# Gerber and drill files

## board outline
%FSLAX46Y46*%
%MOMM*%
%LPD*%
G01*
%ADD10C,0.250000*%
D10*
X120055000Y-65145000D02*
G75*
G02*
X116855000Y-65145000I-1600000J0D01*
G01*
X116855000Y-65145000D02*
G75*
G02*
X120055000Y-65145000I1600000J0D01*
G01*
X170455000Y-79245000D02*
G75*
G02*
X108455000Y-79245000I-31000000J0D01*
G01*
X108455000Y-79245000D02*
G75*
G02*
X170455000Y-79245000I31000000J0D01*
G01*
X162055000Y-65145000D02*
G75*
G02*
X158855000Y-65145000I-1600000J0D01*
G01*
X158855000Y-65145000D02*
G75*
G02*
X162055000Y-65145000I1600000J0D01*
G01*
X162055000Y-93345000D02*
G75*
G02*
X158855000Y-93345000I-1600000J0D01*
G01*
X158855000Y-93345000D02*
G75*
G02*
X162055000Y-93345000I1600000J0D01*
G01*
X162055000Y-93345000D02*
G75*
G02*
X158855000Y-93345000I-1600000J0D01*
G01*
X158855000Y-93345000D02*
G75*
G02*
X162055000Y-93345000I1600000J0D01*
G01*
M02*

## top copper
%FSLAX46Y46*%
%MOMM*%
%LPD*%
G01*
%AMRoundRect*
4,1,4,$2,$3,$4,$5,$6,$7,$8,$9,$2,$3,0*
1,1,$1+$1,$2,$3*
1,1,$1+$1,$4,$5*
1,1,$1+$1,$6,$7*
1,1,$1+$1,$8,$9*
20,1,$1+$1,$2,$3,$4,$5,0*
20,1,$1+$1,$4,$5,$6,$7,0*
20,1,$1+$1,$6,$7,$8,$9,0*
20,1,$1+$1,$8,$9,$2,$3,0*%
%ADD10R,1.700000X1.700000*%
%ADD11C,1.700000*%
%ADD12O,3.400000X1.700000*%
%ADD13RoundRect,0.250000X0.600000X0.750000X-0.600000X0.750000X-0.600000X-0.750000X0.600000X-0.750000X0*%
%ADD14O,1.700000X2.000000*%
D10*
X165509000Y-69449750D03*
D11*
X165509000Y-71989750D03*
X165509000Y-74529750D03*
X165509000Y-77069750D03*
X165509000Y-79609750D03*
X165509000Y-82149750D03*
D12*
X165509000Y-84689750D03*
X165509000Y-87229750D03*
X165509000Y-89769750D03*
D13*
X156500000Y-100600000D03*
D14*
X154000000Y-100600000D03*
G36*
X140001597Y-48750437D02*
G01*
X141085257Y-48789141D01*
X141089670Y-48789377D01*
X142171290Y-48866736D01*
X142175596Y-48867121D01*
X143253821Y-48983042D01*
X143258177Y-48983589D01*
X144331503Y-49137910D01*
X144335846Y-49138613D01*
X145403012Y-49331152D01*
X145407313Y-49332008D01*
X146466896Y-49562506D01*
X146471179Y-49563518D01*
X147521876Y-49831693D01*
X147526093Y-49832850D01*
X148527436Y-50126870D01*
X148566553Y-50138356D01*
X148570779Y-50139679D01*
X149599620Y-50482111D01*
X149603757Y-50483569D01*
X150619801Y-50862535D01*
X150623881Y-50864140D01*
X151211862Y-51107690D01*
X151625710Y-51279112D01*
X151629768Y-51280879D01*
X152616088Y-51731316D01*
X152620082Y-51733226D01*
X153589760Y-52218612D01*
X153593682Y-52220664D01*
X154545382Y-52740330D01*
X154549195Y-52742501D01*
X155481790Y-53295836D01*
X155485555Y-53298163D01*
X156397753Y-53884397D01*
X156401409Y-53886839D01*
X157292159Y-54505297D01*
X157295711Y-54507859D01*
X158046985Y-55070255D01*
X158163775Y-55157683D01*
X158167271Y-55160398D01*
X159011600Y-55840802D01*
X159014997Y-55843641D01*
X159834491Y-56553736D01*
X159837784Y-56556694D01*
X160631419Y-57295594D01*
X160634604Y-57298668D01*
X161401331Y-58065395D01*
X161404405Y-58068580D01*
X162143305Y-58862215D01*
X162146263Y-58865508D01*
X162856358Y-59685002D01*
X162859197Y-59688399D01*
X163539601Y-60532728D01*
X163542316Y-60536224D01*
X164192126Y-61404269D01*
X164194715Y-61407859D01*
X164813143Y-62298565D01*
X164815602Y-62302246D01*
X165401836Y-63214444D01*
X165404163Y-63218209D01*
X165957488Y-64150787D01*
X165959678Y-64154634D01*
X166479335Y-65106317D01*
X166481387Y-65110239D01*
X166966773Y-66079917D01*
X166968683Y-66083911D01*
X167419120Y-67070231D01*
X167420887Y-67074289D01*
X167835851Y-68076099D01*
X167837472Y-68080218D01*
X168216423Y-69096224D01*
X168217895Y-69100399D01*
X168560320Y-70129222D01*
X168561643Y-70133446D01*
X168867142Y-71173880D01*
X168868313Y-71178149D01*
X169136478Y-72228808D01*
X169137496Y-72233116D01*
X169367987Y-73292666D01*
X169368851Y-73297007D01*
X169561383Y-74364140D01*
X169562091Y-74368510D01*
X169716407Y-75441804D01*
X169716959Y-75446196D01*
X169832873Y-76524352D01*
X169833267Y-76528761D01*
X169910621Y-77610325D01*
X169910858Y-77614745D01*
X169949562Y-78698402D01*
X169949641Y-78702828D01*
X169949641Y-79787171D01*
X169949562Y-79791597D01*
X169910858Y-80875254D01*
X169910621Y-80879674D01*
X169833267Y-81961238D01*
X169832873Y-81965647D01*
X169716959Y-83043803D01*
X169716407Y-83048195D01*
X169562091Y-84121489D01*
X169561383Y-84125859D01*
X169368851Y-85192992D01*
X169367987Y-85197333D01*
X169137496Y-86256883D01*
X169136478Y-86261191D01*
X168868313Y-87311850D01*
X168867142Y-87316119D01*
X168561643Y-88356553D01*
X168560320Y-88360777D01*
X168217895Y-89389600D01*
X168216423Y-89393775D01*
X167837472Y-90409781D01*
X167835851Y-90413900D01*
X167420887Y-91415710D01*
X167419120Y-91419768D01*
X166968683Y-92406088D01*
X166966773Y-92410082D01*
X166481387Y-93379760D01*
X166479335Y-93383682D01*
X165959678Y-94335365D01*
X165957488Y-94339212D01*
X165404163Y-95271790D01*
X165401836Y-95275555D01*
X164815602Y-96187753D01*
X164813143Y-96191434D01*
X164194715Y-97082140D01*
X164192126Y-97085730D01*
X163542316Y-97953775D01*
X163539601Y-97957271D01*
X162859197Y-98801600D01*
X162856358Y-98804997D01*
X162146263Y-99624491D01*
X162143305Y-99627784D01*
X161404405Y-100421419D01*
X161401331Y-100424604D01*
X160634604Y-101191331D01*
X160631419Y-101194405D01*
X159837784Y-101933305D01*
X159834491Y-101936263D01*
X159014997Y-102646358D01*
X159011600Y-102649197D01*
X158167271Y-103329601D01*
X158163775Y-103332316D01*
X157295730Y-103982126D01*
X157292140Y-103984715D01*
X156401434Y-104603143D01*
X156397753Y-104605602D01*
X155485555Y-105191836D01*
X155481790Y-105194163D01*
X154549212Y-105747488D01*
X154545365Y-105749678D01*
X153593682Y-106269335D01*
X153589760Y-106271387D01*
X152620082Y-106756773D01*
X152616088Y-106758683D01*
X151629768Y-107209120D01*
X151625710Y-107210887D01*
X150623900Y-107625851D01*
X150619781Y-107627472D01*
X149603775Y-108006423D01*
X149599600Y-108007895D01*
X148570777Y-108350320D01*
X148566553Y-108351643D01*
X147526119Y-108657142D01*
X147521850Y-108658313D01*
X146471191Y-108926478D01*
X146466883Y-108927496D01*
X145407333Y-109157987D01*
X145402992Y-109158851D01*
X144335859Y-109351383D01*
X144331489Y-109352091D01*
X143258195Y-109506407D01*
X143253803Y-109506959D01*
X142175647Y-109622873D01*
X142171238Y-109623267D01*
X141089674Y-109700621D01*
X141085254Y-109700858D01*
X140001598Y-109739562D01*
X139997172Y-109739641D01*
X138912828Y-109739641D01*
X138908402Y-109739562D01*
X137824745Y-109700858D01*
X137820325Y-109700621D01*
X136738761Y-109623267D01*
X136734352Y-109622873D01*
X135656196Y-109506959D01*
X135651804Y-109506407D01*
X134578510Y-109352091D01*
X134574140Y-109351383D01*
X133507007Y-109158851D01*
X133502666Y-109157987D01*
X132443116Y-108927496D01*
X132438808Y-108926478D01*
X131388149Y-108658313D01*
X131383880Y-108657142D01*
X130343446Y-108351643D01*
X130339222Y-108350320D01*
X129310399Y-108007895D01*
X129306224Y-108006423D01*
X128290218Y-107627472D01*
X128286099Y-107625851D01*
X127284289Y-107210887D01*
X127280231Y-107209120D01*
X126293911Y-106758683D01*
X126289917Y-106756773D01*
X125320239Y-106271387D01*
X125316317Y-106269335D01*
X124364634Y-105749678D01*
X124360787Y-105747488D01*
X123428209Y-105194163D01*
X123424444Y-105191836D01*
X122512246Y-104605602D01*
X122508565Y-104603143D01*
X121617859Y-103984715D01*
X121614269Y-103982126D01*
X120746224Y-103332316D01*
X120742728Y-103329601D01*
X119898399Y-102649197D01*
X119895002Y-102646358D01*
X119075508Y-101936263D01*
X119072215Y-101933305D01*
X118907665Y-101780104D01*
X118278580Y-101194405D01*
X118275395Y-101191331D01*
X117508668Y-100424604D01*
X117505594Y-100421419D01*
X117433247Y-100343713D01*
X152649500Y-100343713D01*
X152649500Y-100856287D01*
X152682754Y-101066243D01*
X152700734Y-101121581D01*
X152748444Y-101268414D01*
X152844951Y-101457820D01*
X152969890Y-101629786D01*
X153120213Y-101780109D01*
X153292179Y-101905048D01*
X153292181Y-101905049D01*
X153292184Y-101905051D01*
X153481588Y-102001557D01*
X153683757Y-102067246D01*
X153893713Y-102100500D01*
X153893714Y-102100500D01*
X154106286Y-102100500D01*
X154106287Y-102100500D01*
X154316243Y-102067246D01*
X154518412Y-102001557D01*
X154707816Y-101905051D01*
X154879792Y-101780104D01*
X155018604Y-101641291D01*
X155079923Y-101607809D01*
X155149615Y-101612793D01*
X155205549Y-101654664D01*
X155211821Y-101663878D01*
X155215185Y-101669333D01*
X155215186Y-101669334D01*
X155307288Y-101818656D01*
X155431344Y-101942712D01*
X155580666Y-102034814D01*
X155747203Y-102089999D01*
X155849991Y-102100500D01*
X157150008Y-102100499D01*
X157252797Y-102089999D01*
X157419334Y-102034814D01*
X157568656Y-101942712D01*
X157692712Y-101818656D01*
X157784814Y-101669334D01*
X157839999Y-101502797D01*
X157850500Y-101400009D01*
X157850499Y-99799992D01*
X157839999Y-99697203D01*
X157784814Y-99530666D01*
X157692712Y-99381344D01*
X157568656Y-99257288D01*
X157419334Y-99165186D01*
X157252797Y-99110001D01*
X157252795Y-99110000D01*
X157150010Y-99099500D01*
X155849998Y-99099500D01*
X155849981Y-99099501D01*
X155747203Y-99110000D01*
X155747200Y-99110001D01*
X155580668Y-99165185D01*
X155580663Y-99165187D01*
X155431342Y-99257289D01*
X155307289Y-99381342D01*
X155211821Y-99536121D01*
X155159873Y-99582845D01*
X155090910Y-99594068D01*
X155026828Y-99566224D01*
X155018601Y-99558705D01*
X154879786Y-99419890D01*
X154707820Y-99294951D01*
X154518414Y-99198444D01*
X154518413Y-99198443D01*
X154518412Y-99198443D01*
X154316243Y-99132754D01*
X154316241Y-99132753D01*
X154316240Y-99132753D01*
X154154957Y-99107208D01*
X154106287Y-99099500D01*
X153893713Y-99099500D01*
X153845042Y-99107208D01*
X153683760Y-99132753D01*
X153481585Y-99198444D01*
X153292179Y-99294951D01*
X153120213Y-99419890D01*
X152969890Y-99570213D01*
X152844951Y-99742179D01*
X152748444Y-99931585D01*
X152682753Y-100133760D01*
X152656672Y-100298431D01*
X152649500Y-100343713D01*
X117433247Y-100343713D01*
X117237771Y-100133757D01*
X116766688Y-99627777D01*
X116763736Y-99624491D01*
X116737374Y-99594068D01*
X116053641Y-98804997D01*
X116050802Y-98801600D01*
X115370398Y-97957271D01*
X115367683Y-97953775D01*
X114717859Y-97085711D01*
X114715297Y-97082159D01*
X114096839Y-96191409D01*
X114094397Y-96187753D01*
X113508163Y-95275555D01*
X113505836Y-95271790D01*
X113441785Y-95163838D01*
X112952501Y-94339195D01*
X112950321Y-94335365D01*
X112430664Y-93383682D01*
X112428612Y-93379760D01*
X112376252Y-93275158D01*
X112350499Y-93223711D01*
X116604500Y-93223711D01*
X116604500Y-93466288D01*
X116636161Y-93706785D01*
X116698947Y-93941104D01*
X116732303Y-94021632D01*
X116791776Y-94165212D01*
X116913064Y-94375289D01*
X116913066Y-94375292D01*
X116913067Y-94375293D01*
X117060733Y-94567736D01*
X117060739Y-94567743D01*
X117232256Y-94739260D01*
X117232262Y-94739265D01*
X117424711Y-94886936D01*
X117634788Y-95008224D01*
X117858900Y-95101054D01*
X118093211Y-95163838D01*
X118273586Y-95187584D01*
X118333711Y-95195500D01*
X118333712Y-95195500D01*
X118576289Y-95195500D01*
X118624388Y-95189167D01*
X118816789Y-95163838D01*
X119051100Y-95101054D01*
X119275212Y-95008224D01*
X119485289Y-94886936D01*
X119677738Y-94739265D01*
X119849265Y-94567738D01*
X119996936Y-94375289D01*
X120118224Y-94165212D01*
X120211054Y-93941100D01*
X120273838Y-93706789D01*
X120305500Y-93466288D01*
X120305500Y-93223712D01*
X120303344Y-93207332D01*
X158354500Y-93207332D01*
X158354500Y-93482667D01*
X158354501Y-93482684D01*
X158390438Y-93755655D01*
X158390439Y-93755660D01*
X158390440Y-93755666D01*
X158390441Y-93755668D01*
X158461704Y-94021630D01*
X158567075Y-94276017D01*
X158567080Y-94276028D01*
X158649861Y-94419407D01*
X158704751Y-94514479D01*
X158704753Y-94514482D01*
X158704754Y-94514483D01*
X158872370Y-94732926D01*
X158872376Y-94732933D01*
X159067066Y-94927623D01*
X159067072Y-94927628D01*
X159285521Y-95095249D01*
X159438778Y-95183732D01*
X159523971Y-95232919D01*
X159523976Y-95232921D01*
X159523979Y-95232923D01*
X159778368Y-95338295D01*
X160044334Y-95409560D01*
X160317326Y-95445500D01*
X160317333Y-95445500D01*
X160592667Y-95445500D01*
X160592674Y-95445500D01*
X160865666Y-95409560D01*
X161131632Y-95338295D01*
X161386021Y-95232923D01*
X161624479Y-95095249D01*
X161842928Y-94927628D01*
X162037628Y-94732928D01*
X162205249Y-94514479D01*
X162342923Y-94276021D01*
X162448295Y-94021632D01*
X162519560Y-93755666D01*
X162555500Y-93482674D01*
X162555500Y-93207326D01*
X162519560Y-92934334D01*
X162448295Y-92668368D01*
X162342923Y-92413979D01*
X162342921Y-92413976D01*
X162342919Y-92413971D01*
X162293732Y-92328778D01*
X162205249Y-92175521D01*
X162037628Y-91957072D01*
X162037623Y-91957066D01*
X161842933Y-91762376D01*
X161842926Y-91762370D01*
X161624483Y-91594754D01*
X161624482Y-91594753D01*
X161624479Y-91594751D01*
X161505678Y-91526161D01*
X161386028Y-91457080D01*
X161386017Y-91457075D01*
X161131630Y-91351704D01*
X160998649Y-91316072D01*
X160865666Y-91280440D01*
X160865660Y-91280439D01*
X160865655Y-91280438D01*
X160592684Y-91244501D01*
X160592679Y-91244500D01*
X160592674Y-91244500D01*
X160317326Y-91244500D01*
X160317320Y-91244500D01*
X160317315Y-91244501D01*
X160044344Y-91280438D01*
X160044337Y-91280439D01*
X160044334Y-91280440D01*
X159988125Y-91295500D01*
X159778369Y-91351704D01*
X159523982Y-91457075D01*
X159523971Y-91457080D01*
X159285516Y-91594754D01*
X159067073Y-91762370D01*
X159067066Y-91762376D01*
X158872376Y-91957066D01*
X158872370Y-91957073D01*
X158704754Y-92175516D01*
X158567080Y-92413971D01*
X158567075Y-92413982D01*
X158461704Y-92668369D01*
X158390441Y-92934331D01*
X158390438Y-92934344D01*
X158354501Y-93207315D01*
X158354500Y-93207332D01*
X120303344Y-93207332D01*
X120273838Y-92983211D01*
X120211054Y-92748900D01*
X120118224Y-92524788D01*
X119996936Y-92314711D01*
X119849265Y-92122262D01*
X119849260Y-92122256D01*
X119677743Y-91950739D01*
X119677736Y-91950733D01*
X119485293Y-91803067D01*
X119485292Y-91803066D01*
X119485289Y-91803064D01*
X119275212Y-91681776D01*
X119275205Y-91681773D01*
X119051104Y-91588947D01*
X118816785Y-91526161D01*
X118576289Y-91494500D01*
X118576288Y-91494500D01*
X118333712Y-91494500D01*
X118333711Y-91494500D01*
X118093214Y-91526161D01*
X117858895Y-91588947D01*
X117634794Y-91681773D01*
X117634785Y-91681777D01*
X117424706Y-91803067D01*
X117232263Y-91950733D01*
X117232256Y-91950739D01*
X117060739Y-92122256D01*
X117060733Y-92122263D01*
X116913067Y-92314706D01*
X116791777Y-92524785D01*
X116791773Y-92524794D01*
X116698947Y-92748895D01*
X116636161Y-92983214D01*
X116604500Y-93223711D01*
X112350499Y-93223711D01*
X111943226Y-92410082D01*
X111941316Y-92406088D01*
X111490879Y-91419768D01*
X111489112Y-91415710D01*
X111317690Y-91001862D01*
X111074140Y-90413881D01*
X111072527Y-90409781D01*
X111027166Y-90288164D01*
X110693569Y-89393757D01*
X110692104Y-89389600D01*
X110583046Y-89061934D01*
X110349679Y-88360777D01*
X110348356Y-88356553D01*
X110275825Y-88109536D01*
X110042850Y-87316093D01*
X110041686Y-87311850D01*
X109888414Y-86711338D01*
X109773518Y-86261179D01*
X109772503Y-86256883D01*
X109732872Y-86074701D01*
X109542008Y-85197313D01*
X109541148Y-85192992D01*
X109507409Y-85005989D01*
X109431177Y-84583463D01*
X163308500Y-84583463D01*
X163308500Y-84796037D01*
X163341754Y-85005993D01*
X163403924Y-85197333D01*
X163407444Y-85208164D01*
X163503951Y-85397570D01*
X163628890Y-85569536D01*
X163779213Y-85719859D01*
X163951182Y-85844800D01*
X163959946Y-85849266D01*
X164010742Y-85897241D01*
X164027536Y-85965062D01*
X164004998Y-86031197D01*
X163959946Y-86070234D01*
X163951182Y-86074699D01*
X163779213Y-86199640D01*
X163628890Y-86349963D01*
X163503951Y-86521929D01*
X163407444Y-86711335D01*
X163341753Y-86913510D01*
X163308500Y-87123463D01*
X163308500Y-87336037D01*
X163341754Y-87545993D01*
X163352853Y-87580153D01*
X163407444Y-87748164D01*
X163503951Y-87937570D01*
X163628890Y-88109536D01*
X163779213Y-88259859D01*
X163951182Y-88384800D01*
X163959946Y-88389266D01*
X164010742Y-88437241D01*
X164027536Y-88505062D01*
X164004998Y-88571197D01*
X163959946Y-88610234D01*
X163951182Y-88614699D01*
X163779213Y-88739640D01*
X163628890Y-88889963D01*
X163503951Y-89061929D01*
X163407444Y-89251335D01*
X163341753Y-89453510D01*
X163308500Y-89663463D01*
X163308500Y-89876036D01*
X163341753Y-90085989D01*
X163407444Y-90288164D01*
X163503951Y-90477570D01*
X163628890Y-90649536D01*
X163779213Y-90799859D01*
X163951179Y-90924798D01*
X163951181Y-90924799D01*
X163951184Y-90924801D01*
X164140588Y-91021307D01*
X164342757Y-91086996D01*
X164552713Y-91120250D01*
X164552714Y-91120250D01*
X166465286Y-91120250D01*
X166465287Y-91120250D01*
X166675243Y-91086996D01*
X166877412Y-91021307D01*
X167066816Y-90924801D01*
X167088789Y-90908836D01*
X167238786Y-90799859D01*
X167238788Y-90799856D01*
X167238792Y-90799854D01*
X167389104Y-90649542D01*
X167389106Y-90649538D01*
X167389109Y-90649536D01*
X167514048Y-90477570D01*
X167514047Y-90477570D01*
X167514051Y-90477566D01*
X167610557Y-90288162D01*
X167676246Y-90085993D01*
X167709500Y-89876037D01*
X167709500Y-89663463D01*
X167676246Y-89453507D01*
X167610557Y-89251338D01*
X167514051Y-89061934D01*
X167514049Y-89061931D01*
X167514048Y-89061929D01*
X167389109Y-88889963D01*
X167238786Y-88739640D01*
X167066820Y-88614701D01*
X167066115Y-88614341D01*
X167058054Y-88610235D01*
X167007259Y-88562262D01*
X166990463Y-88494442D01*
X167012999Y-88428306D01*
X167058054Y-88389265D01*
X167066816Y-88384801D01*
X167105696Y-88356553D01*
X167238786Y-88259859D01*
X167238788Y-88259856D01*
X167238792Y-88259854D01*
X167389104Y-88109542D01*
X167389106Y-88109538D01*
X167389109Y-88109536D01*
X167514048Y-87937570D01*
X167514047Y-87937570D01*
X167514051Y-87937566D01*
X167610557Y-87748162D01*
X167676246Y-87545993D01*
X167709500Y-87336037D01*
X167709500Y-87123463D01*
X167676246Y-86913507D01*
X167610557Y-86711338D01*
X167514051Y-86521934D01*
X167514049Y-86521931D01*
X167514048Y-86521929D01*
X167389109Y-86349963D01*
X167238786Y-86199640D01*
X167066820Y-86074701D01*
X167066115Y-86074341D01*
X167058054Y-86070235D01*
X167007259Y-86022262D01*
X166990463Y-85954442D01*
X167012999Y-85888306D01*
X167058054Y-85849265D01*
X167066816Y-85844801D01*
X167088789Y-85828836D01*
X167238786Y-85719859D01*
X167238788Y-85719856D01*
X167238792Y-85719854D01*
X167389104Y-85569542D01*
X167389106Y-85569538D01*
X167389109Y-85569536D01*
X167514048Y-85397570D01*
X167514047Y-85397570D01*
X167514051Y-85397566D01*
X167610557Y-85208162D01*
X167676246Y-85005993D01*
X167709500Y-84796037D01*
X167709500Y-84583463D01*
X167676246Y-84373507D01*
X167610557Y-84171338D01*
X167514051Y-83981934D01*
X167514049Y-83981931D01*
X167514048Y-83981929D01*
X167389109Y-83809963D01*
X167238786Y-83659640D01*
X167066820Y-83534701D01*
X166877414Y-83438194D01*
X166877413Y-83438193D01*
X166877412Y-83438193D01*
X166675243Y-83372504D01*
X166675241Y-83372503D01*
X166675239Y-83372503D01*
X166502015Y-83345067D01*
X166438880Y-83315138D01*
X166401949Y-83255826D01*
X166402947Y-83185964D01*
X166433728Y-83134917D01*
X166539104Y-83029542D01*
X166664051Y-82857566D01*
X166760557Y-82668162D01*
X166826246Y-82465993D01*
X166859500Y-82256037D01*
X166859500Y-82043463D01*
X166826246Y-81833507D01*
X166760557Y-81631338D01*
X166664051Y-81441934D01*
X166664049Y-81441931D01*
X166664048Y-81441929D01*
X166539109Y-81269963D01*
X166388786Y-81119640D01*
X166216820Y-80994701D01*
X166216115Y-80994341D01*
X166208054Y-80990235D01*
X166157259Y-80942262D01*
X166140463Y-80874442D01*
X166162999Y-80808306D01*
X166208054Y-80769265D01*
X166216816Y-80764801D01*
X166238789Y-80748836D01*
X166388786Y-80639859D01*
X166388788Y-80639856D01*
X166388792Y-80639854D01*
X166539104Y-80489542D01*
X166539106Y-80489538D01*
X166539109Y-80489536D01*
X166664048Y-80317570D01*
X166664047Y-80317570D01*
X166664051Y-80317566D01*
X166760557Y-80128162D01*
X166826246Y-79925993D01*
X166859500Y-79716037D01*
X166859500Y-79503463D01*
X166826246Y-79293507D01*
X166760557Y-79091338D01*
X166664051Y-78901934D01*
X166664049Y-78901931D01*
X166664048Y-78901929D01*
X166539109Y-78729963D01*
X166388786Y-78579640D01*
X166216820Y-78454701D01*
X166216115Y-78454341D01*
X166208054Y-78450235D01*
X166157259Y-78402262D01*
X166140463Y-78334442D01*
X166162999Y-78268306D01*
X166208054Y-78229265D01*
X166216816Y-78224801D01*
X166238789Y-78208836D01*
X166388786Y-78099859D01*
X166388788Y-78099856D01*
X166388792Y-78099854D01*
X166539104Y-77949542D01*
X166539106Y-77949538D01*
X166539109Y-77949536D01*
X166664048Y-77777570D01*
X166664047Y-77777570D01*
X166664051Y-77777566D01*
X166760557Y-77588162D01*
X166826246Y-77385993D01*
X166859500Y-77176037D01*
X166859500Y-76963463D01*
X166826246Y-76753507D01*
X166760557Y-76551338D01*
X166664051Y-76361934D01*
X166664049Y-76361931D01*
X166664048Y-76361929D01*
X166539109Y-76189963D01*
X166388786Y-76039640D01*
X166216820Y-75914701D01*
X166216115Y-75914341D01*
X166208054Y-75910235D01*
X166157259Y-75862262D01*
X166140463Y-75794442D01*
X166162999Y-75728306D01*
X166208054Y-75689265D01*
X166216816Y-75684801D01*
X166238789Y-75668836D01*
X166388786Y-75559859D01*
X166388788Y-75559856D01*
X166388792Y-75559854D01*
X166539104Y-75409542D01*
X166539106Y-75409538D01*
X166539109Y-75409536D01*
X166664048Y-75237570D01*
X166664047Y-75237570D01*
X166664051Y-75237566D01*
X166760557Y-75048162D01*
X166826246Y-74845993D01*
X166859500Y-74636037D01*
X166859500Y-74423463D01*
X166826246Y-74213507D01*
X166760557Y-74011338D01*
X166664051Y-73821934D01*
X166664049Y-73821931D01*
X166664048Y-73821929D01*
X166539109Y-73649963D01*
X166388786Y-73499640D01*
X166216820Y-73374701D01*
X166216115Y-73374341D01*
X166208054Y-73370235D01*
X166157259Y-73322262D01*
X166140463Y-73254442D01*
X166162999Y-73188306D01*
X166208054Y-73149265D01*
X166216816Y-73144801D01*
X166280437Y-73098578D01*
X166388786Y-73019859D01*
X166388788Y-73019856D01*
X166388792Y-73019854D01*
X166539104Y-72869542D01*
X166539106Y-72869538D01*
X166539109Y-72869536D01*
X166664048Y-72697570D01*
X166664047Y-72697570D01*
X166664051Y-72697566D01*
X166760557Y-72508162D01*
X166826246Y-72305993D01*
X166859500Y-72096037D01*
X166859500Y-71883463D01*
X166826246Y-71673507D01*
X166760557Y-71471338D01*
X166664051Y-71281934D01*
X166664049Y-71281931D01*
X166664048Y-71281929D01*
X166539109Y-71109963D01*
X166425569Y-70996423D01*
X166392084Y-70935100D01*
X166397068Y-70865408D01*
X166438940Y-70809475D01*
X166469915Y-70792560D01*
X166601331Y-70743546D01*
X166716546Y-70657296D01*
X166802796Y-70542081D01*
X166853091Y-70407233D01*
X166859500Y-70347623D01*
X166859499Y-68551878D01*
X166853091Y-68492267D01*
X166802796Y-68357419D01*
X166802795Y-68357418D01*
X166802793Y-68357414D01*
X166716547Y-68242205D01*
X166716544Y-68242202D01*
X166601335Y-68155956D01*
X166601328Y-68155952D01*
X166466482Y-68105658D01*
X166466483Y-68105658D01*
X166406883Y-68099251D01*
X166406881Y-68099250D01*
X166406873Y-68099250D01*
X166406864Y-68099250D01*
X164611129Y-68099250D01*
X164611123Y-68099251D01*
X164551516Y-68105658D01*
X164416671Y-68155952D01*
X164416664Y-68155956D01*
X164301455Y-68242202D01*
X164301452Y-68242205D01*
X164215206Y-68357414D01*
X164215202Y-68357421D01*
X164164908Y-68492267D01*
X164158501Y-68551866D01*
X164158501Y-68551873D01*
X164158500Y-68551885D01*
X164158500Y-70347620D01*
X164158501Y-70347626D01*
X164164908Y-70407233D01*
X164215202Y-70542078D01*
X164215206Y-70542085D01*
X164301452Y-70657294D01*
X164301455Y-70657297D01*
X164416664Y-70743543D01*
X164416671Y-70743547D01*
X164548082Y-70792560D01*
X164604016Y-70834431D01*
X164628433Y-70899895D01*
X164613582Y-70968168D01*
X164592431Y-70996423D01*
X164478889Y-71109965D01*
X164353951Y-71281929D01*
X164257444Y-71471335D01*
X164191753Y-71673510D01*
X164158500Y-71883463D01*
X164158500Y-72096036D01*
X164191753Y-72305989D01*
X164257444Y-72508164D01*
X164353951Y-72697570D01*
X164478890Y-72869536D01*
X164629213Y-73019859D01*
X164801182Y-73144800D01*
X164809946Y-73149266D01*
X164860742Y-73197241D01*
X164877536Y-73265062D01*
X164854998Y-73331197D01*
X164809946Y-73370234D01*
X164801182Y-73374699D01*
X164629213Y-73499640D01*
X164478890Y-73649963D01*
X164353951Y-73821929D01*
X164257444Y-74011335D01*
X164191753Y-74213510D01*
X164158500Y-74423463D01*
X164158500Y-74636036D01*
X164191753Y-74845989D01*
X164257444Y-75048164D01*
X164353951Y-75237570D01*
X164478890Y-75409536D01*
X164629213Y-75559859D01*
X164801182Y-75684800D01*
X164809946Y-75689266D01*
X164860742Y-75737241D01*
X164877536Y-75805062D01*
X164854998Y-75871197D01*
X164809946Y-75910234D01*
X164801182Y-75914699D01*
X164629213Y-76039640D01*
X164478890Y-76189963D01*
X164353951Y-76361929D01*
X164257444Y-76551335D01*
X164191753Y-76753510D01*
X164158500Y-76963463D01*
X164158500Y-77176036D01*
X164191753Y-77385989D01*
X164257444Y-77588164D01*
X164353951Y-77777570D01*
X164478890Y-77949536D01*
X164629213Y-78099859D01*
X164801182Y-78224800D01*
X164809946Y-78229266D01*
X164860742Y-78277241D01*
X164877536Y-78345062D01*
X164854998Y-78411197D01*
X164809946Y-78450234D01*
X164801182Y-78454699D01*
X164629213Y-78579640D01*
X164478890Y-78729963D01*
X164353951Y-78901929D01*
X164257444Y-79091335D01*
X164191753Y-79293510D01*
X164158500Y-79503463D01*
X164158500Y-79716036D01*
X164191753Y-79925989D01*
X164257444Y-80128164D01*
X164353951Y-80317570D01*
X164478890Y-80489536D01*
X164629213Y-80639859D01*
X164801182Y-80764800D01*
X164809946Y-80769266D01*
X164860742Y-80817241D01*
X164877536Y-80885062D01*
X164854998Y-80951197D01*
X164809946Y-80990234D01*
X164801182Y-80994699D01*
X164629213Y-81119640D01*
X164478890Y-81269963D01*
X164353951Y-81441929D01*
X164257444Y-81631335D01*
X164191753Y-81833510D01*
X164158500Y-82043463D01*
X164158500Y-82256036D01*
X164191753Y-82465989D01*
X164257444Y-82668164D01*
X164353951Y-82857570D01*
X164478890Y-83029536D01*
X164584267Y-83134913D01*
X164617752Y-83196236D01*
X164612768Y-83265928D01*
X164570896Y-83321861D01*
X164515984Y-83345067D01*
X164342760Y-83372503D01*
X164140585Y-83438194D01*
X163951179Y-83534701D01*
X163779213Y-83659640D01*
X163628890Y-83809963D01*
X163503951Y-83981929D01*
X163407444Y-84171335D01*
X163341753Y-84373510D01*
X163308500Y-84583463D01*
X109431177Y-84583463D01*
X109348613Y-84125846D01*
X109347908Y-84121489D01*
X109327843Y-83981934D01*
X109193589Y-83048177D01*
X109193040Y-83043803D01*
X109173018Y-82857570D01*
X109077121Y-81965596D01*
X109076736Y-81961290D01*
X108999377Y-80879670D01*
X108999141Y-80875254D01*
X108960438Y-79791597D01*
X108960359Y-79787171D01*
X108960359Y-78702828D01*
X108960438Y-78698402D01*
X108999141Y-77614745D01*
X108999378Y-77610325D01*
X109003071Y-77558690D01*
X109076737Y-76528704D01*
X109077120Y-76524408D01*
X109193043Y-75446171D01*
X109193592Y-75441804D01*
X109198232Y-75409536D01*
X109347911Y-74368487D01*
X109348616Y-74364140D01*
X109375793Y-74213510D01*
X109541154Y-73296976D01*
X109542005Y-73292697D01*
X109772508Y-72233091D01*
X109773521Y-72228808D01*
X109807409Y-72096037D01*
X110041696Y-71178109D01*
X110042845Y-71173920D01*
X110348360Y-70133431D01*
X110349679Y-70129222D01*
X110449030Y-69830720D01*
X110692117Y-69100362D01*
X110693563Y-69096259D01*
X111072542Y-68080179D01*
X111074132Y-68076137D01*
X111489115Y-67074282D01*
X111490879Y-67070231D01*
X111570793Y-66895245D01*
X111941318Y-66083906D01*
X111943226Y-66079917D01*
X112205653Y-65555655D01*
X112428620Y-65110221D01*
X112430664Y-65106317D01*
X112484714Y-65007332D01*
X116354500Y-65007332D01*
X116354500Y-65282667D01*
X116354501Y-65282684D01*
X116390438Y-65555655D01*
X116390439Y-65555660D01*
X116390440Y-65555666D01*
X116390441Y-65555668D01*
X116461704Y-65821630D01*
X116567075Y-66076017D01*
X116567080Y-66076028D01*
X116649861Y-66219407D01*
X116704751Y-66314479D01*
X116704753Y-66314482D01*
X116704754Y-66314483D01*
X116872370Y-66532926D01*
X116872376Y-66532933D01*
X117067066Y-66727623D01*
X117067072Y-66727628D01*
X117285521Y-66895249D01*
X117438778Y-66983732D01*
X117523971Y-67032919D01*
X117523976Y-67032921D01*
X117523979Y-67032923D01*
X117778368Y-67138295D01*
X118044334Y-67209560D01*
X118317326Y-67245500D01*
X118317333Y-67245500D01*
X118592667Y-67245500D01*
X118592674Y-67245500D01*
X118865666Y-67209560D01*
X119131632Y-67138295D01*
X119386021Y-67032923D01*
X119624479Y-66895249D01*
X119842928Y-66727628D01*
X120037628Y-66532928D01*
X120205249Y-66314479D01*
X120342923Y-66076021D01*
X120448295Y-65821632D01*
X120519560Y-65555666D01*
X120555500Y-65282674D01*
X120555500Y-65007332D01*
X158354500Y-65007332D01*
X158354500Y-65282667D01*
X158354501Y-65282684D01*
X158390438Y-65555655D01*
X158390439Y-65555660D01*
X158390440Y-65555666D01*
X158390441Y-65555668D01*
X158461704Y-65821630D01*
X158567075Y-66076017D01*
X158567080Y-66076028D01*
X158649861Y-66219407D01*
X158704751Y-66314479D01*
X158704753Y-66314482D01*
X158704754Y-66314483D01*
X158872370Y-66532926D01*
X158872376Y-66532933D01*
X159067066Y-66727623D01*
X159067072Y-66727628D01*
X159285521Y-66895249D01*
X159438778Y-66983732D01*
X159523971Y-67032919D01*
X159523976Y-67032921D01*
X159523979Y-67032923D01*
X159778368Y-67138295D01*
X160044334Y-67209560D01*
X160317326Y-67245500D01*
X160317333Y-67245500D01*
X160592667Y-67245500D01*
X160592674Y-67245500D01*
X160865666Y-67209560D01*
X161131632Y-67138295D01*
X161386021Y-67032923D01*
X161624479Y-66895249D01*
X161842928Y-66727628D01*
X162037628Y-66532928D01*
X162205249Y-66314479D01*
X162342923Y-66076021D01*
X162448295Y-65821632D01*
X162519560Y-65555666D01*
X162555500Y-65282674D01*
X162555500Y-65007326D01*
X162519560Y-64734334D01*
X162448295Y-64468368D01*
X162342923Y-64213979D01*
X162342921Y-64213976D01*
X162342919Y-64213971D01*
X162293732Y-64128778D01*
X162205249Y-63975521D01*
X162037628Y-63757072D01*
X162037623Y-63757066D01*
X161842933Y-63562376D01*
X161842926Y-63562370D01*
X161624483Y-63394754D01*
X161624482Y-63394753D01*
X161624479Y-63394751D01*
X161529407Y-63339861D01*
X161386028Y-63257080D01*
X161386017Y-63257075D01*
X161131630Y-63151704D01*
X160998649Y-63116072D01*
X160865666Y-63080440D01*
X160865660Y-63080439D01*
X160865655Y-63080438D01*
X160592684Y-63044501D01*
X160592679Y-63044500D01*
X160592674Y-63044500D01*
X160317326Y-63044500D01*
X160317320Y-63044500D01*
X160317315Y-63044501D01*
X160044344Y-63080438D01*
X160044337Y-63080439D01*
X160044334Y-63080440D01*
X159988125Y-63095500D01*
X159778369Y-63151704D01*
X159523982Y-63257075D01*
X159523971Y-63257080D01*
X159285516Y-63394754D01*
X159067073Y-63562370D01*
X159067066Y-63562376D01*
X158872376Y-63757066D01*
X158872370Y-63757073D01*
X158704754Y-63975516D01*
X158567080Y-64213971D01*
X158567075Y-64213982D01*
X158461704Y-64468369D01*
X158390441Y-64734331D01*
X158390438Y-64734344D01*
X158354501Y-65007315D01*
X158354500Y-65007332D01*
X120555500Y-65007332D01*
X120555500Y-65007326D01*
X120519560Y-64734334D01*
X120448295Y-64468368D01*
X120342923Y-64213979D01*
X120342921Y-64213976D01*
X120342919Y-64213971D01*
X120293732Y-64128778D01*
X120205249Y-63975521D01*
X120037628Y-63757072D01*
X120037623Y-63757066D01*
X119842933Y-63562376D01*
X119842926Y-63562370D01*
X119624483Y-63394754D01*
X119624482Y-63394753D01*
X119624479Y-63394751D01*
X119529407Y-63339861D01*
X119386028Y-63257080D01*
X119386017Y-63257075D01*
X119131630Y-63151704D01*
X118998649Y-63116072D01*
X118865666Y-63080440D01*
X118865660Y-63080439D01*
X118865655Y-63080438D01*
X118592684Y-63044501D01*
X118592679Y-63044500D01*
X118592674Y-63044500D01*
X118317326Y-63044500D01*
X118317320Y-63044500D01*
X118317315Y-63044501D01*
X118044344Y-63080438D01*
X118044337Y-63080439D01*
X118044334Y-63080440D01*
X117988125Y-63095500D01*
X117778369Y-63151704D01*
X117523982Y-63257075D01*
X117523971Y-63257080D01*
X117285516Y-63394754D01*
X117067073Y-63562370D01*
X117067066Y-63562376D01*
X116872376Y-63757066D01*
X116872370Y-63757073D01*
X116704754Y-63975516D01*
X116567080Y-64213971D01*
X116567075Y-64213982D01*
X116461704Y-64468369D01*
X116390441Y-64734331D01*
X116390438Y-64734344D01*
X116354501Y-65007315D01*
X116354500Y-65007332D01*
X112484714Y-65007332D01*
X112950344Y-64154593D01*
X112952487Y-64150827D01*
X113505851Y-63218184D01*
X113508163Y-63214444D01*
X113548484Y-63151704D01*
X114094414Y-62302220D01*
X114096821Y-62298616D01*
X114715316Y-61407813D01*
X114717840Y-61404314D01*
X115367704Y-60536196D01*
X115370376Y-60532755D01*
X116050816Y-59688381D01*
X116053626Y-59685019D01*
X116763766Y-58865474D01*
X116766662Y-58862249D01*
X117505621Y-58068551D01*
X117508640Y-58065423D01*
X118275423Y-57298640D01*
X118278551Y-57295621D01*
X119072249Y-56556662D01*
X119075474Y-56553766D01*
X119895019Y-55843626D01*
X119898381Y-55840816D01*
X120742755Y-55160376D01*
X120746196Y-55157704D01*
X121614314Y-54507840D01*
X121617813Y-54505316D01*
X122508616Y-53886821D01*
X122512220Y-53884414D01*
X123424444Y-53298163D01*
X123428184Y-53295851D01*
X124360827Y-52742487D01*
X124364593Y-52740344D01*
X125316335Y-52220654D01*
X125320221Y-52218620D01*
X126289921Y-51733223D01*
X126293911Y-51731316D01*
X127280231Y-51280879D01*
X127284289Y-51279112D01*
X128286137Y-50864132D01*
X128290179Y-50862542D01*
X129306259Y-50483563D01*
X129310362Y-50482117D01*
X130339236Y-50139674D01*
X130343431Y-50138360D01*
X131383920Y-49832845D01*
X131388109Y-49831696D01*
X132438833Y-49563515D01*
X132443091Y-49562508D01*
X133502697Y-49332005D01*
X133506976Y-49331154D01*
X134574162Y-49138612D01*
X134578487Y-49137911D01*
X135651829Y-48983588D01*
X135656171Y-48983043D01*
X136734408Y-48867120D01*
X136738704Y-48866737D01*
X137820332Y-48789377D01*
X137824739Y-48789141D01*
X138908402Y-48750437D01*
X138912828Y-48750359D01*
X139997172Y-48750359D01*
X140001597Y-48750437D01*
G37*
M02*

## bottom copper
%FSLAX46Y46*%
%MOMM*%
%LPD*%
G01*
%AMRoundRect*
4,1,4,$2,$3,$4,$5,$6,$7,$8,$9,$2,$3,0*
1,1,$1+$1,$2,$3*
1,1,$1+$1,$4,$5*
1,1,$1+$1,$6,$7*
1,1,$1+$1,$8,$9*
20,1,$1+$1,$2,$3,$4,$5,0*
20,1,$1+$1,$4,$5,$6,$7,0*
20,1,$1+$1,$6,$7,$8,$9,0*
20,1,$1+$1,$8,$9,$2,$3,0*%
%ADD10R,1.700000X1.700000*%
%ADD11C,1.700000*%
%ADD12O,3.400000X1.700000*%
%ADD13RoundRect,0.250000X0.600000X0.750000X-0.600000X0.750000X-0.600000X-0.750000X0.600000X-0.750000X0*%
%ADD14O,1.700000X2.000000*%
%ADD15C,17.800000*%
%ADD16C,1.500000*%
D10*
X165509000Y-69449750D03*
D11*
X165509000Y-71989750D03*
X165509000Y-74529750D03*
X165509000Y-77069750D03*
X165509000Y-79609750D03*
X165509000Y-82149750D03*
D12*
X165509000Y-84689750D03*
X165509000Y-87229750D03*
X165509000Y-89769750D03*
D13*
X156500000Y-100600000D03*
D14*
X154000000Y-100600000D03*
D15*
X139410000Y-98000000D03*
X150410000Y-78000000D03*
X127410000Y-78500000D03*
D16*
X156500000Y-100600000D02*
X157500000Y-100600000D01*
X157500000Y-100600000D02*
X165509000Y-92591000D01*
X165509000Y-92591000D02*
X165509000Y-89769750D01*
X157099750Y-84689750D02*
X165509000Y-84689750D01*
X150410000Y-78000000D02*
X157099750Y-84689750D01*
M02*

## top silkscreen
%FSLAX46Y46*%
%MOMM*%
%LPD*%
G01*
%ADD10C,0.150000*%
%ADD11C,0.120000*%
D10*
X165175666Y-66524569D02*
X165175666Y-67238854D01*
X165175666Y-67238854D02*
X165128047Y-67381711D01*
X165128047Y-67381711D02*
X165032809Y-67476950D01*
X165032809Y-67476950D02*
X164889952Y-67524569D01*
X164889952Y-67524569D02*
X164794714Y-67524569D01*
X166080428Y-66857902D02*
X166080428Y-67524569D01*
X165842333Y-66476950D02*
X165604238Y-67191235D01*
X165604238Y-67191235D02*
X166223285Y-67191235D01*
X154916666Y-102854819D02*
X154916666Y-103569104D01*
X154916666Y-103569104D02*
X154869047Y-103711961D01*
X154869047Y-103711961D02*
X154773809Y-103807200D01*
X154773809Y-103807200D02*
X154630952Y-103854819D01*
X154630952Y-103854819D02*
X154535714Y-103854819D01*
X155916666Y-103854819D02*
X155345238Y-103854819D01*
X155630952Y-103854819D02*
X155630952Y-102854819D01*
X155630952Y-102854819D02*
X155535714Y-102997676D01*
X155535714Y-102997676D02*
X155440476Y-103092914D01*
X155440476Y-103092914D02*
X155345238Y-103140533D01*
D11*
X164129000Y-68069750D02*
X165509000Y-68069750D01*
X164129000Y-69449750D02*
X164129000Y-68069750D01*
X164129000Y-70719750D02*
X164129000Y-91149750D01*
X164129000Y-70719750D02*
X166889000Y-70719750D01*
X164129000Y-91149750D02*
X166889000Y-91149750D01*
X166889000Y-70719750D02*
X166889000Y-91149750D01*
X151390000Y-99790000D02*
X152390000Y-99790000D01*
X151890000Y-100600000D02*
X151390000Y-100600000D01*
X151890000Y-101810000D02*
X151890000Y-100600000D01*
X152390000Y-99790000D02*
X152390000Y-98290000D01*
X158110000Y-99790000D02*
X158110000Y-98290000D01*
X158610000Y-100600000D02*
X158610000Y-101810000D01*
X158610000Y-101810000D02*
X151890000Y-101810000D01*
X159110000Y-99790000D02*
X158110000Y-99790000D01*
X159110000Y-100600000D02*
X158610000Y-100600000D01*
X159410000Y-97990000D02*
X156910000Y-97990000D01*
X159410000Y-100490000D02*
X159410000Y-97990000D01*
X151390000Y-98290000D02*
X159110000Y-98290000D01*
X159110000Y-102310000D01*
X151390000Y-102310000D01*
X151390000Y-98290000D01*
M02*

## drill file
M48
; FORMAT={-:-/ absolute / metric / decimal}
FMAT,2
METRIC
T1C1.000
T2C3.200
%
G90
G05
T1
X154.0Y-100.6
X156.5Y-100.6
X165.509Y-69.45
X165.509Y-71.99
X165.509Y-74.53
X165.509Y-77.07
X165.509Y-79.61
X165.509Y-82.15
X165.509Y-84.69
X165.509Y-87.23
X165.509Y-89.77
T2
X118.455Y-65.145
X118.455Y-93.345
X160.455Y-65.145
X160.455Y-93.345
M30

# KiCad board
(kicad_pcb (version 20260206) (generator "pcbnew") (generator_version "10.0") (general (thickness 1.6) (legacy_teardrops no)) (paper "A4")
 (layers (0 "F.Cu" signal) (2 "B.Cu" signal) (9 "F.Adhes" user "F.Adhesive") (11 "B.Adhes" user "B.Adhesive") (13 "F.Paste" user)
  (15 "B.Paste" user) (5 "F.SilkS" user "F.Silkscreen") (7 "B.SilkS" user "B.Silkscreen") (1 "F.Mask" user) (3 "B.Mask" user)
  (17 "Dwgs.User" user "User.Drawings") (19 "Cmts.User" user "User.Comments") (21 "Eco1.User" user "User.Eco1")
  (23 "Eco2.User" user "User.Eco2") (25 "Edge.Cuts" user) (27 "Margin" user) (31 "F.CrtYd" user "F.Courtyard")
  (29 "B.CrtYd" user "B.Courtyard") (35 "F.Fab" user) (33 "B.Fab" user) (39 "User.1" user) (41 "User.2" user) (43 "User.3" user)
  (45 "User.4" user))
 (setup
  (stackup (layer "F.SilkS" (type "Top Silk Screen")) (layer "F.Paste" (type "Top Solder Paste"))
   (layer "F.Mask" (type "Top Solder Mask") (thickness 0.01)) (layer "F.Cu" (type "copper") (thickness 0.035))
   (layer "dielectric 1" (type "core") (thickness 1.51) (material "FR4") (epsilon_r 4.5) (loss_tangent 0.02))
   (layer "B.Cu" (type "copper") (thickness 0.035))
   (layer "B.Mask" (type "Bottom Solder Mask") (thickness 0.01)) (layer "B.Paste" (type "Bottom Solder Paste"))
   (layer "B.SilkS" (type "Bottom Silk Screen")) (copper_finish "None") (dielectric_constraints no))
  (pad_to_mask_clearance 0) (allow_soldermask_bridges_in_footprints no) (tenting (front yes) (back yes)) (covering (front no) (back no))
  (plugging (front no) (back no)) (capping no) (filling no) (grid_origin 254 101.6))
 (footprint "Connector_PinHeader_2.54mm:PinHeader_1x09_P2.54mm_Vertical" (layer "F.Cu") (at 165.509 69.44975)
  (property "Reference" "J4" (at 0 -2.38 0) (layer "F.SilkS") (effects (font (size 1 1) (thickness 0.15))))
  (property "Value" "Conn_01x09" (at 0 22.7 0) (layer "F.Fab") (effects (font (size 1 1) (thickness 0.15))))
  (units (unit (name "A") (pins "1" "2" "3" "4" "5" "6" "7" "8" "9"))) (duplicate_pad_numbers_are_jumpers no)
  (fp_line (start -1.38 -1.38) (end 0 -1.38) (stroke (width 0.12) (type solid)) (layer "F.SilkS"))
  (fp_line (start -1.38 0) (end -1.38 -1.38) (stroke (width 0.12) (type solid)) (layer "F.SilkS"))
  (fp_line (start -1.38 1.27) (end -1.38 21.7) (stroke (width 0.12) (type solid)) (layer "F.SilkS"))
  (fp_line (start -1.38 1.27) (end 1.38 1.27) (stroke (width 0.12) (type solid)) (layer "F.SilkS"))
  (fp_line (start -1.38 21.7) (end 1.38 21.7) (stroke (width 0.12) (type solid)) (layer "F.SilkS"))
  (fp_line (start 1.38 1.27) (end 1.38 21.7) (stroke (width 0.12) (type solid)) (layer "F.SilkS"))
  (pad "1" thru_hole rect (at 0 0) (size 1.7 1.7) (drill 1) (layers "*.Cu" "*.Mask") (remove_unused_layers no)
   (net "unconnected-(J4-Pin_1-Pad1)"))
  (pad "2" thru_hole circle (at 0 2.54) (size 1.7 1.7) (drill 1) (layers "*.Cu" "*.Mask") (remove_unused_layers no)
   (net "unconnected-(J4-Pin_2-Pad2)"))
  (pad "3" thru_hole circle (at 0 5.08) (size 1.7 1.7) (drill 1) (layers "*.Cu" "*.Mask") (remove_unused_layers no)
   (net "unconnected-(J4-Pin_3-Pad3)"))
  (pad "4" thru_hole circle (at 0 7.62) (size 1.7 1.7) (drill 1) (layers "*.Cu" "*.Mask") (remove_unused_layers no)
   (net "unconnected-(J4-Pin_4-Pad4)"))
  (pad "5" thru_hole circle (at 0 10.16) (size 1.7 1.7) (drill 1) (layers "*.Cu" "*.Mask") (remove_unused_layers no)
   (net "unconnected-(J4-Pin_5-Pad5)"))
  (pad "6" thru_hole circle (at 0 12.7) (size 1.7 1.7) (drill 1) (layers "*.Cu" "*.Mask") (remove_unused_layers no)
   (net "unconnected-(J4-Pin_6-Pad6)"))
  (pad "7" thru_hole oval (at 0 15.24) (size 3.4 1.7) (drill 1) (layers "*.Cu" "*.Mask") (remove_unused_layers no) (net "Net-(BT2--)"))
  (pad "8" thru_hole oval (at 0 17.78) (size 3.4 1.7) (drill 1) (layers "*.Cu" "*.Mask") (remove_unused_layers no)
   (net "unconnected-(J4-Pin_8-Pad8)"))
  (pad "9" thru_hole oval (at 0 20.32) (size 3.4 1.7) (drill 1) (layers "*.Cu" "*.Mask") (remove_unused_layers no) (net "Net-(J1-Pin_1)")))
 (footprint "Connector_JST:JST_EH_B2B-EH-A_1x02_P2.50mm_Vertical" (layer "F.Cu") (at 156.5 100.6 180)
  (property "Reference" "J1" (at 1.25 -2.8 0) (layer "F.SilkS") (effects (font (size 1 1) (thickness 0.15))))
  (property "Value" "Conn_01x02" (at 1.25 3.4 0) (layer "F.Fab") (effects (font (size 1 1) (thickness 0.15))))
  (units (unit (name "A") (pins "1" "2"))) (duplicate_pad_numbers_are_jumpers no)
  (fp_line (start 5.11 0.81) (end 4.11 0.81) (stroke (width 0.12) (type solid)) (layer "F.SilkS"))
  (fp_line (start 4.61 0) (end 5.11 0) (stroke (width 0.12) (type solid)) (layer "F.SilkS"))
  (fp_line (start 4.61 -1.21) (end 4.61 0) (stroke (width 0.12) (type solid)) (layer "F.SilkS"))
  (fp_line (start 4.11 0.81) (end 4.11 2.31) (stroke (width 0.12) (type solid)) (layer "F.SilkS"))
  (fp_line (start -1.61 0.81) (end -1.61 2.31) (stroke (width 0.12) (type solid)) (layer "F.SilkS"))
  (fp_line (start -2.11 0) (end -2.11 -1.21) (stroke (width 0.12) (type solid)) (layer "F.SilkS"))
  (fp_line (start -2.11 -1.21) (end 4.61 -1.21) (stroke (width 0.12) (type solid)) (layer "F.SilkS"))
  (fp_line (start -2.61 0.81) (end -1.61 0.81) (stroke (width 0.12) (type solid)) (layer "F.SilkS"))
  (fp_line (start -2.61 0) (end -2.11 0) (stroke (width 0.12) (type solid)) (layer "F.SilkS"))
  (fp_line (start -2.91 2.61) (end -0.41 2.61) (stroke (width 0.12) (type solid)) (layer "F.SilkS"))
  (fp_line (start -2.91 0.11) (end -2.91 2.61) (stroke (width 0.12) (type solid)) (layer "F.SilkS"))
  (fp_rect (start -2.61 -1.71) (end 5.11 2.31) (stroke (width 0.12) (type solid)) (fill no) (layer "F.SilkS"))
  (pad "1" thru_hole roundrect (at 0 0 180) (size 1.7 2) (drill 1) (layers "*.Cu" "*.Mask") (remove_unused_layers no)
   (roundrect_rratio 0.147059) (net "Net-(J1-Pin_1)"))
  (pad "2" thru_hole oval (at 2.5 0 180) (size 1.7 2) (drill 1) (layers "*.Cu" "*.Mask") (remove_unused_layers no)
   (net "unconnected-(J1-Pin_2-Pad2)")))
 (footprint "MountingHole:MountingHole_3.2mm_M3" (layer "B.Cu") (at 118.455 93.345 180)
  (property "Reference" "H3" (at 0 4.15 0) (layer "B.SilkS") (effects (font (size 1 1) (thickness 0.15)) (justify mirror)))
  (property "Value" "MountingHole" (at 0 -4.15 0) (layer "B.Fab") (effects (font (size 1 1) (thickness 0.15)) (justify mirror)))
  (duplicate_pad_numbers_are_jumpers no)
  (pad "" np_thru_hole circle (at 0 0 180) (size 3.2 3.2) (drill 3.2) (layers "*.Cu" "*.Mask")))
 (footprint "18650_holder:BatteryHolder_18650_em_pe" (layer "B.Cu") (at 139.41 98 180)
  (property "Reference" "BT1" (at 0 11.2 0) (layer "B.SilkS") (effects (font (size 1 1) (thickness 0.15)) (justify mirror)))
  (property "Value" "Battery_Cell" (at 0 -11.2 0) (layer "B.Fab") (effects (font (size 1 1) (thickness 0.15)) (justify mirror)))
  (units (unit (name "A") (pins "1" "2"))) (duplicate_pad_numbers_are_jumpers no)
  (pad "2" smd circle (at 0 0 180) (size 17.8 17.8) (layers "B.Cu" "B.Mask") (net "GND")))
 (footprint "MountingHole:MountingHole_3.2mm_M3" (layer "B.Cu") (at 118.455 65.145 180)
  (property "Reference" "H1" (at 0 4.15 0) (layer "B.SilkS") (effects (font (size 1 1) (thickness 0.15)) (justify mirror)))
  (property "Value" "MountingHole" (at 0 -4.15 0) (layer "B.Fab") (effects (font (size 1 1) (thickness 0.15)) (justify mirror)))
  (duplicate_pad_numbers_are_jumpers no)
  (pad "" np_thru_hole circle (at 0 0 180) (size 3.2 3.2) (drill 3.2) (layers "*.Cu" "*.Mask")))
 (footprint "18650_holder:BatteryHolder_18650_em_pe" (layer "B.Cu") (at 150.41 78 180)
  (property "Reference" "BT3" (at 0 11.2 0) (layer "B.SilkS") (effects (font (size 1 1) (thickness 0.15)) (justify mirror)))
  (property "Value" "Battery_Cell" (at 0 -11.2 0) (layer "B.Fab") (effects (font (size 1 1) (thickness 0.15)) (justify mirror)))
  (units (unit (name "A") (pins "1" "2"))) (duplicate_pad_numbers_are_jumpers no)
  (pad "2" smd circle (at 0 0 180) (size 17.8 17.8) (layers "B.Cu" "B.Mask") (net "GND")))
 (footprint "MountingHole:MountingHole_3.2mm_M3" (layer "B.Cu") (at 160.455 65.145 180)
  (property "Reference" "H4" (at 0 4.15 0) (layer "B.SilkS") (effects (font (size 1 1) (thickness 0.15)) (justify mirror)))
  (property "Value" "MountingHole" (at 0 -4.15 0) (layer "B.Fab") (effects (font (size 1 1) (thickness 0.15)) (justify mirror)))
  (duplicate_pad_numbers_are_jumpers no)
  (pad "" np_thru_hole circle (at 0 0 180) (size 3.2 3.2) (drill 3.2) (layers "*.Cu" "*.Mask")))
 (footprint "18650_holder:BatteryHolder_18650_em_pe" (layer "B.Cu") (at 127.41 78.5 180)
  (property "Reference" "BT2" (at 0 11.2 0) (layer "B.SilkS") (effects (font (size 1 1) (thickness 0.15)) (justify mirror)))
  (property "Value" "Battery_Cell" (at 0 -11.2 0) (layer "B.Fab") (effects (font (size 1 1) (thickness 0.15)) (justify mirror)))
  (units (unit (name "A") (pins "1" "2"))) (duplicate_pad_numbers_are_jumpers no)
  (pad "2" smd circle (at 0 0 180) (size 17.8 17.8) (layers "B.Cu" "B.Mask") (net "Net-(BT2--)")))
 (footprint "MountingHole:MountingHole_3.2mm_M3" (layer "B.Cu") (at 160.455 93.345 180)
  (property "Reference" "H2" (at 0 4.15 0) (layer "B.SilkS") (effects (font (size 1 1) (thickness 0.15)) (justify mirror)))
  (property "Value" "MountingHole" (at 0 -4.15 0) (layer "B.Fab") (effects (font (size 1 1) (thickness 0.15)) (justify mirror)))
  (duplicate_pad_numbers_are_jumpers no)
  (pad "" np_thru_hole circle (at 0 0 180) (size 3.2 3.2) (drill 3.2) (layers "*.Cu" "*.Mask")))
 (gr_circle (center 118.455 65.145) (end 116.855 65.145) (stroke (width 0.25) (type default)) (fill no) (layer "Edge.Cuts"))
 (gr_circle (center 139.455 79.245) (end 170.455 79.245) (stroke (width 0.25) (type solid)) (fill no) (layer "Edge.Cuts"))
 (gr_circle (center 160.455 65.145) (end 158.855 65.145) (stroke (width 0.25) (type default)) (fill no) (layer "Edge.Cuts"))
 (gr_circle (center 160.455 93.345) (end 158.855 93.345) (stroke (width 0.25) (type default)) (fill no) (layer "Edge.Cuts"))
 (gr_circle (center 160.455 93.345) (end 162.055 93.345) (stroke (width 0.25) (type default)) (fill no) (layer "Edge.Cuts"))
 (segment (start 156.5 100.6) (end 157.5 100.6) (width 1.5) (layer "B.Cu") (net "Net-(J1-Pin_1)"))
 (segment (start 157.5 100.6) (end 165.509 92.591) (width 1.5) (layer "B.Cu") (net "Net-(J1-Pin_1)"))
 (segment (start 165.509 92.591) (end 165.509 89.76975) (width 1.5) (layer "B.Cu") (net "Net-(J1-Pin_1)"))
 (segment (start 157.09975 84.68975) (end 165.509 84.68975) (width 1.5) (layer "B.Cu") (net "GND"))
 (segment (start 150.41 78) (end 157.09975 84.68975) (width 1.5) (layer "B.Cu") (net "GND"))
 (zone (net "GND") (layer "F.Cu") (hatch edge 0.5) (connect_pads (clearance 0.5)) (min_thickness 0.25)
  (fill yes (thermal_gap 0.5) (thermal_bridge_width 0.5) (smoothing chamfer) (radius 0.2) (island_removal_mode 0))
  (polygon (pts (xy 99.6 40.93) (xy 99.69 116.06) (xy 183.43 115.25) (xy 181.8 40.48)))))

